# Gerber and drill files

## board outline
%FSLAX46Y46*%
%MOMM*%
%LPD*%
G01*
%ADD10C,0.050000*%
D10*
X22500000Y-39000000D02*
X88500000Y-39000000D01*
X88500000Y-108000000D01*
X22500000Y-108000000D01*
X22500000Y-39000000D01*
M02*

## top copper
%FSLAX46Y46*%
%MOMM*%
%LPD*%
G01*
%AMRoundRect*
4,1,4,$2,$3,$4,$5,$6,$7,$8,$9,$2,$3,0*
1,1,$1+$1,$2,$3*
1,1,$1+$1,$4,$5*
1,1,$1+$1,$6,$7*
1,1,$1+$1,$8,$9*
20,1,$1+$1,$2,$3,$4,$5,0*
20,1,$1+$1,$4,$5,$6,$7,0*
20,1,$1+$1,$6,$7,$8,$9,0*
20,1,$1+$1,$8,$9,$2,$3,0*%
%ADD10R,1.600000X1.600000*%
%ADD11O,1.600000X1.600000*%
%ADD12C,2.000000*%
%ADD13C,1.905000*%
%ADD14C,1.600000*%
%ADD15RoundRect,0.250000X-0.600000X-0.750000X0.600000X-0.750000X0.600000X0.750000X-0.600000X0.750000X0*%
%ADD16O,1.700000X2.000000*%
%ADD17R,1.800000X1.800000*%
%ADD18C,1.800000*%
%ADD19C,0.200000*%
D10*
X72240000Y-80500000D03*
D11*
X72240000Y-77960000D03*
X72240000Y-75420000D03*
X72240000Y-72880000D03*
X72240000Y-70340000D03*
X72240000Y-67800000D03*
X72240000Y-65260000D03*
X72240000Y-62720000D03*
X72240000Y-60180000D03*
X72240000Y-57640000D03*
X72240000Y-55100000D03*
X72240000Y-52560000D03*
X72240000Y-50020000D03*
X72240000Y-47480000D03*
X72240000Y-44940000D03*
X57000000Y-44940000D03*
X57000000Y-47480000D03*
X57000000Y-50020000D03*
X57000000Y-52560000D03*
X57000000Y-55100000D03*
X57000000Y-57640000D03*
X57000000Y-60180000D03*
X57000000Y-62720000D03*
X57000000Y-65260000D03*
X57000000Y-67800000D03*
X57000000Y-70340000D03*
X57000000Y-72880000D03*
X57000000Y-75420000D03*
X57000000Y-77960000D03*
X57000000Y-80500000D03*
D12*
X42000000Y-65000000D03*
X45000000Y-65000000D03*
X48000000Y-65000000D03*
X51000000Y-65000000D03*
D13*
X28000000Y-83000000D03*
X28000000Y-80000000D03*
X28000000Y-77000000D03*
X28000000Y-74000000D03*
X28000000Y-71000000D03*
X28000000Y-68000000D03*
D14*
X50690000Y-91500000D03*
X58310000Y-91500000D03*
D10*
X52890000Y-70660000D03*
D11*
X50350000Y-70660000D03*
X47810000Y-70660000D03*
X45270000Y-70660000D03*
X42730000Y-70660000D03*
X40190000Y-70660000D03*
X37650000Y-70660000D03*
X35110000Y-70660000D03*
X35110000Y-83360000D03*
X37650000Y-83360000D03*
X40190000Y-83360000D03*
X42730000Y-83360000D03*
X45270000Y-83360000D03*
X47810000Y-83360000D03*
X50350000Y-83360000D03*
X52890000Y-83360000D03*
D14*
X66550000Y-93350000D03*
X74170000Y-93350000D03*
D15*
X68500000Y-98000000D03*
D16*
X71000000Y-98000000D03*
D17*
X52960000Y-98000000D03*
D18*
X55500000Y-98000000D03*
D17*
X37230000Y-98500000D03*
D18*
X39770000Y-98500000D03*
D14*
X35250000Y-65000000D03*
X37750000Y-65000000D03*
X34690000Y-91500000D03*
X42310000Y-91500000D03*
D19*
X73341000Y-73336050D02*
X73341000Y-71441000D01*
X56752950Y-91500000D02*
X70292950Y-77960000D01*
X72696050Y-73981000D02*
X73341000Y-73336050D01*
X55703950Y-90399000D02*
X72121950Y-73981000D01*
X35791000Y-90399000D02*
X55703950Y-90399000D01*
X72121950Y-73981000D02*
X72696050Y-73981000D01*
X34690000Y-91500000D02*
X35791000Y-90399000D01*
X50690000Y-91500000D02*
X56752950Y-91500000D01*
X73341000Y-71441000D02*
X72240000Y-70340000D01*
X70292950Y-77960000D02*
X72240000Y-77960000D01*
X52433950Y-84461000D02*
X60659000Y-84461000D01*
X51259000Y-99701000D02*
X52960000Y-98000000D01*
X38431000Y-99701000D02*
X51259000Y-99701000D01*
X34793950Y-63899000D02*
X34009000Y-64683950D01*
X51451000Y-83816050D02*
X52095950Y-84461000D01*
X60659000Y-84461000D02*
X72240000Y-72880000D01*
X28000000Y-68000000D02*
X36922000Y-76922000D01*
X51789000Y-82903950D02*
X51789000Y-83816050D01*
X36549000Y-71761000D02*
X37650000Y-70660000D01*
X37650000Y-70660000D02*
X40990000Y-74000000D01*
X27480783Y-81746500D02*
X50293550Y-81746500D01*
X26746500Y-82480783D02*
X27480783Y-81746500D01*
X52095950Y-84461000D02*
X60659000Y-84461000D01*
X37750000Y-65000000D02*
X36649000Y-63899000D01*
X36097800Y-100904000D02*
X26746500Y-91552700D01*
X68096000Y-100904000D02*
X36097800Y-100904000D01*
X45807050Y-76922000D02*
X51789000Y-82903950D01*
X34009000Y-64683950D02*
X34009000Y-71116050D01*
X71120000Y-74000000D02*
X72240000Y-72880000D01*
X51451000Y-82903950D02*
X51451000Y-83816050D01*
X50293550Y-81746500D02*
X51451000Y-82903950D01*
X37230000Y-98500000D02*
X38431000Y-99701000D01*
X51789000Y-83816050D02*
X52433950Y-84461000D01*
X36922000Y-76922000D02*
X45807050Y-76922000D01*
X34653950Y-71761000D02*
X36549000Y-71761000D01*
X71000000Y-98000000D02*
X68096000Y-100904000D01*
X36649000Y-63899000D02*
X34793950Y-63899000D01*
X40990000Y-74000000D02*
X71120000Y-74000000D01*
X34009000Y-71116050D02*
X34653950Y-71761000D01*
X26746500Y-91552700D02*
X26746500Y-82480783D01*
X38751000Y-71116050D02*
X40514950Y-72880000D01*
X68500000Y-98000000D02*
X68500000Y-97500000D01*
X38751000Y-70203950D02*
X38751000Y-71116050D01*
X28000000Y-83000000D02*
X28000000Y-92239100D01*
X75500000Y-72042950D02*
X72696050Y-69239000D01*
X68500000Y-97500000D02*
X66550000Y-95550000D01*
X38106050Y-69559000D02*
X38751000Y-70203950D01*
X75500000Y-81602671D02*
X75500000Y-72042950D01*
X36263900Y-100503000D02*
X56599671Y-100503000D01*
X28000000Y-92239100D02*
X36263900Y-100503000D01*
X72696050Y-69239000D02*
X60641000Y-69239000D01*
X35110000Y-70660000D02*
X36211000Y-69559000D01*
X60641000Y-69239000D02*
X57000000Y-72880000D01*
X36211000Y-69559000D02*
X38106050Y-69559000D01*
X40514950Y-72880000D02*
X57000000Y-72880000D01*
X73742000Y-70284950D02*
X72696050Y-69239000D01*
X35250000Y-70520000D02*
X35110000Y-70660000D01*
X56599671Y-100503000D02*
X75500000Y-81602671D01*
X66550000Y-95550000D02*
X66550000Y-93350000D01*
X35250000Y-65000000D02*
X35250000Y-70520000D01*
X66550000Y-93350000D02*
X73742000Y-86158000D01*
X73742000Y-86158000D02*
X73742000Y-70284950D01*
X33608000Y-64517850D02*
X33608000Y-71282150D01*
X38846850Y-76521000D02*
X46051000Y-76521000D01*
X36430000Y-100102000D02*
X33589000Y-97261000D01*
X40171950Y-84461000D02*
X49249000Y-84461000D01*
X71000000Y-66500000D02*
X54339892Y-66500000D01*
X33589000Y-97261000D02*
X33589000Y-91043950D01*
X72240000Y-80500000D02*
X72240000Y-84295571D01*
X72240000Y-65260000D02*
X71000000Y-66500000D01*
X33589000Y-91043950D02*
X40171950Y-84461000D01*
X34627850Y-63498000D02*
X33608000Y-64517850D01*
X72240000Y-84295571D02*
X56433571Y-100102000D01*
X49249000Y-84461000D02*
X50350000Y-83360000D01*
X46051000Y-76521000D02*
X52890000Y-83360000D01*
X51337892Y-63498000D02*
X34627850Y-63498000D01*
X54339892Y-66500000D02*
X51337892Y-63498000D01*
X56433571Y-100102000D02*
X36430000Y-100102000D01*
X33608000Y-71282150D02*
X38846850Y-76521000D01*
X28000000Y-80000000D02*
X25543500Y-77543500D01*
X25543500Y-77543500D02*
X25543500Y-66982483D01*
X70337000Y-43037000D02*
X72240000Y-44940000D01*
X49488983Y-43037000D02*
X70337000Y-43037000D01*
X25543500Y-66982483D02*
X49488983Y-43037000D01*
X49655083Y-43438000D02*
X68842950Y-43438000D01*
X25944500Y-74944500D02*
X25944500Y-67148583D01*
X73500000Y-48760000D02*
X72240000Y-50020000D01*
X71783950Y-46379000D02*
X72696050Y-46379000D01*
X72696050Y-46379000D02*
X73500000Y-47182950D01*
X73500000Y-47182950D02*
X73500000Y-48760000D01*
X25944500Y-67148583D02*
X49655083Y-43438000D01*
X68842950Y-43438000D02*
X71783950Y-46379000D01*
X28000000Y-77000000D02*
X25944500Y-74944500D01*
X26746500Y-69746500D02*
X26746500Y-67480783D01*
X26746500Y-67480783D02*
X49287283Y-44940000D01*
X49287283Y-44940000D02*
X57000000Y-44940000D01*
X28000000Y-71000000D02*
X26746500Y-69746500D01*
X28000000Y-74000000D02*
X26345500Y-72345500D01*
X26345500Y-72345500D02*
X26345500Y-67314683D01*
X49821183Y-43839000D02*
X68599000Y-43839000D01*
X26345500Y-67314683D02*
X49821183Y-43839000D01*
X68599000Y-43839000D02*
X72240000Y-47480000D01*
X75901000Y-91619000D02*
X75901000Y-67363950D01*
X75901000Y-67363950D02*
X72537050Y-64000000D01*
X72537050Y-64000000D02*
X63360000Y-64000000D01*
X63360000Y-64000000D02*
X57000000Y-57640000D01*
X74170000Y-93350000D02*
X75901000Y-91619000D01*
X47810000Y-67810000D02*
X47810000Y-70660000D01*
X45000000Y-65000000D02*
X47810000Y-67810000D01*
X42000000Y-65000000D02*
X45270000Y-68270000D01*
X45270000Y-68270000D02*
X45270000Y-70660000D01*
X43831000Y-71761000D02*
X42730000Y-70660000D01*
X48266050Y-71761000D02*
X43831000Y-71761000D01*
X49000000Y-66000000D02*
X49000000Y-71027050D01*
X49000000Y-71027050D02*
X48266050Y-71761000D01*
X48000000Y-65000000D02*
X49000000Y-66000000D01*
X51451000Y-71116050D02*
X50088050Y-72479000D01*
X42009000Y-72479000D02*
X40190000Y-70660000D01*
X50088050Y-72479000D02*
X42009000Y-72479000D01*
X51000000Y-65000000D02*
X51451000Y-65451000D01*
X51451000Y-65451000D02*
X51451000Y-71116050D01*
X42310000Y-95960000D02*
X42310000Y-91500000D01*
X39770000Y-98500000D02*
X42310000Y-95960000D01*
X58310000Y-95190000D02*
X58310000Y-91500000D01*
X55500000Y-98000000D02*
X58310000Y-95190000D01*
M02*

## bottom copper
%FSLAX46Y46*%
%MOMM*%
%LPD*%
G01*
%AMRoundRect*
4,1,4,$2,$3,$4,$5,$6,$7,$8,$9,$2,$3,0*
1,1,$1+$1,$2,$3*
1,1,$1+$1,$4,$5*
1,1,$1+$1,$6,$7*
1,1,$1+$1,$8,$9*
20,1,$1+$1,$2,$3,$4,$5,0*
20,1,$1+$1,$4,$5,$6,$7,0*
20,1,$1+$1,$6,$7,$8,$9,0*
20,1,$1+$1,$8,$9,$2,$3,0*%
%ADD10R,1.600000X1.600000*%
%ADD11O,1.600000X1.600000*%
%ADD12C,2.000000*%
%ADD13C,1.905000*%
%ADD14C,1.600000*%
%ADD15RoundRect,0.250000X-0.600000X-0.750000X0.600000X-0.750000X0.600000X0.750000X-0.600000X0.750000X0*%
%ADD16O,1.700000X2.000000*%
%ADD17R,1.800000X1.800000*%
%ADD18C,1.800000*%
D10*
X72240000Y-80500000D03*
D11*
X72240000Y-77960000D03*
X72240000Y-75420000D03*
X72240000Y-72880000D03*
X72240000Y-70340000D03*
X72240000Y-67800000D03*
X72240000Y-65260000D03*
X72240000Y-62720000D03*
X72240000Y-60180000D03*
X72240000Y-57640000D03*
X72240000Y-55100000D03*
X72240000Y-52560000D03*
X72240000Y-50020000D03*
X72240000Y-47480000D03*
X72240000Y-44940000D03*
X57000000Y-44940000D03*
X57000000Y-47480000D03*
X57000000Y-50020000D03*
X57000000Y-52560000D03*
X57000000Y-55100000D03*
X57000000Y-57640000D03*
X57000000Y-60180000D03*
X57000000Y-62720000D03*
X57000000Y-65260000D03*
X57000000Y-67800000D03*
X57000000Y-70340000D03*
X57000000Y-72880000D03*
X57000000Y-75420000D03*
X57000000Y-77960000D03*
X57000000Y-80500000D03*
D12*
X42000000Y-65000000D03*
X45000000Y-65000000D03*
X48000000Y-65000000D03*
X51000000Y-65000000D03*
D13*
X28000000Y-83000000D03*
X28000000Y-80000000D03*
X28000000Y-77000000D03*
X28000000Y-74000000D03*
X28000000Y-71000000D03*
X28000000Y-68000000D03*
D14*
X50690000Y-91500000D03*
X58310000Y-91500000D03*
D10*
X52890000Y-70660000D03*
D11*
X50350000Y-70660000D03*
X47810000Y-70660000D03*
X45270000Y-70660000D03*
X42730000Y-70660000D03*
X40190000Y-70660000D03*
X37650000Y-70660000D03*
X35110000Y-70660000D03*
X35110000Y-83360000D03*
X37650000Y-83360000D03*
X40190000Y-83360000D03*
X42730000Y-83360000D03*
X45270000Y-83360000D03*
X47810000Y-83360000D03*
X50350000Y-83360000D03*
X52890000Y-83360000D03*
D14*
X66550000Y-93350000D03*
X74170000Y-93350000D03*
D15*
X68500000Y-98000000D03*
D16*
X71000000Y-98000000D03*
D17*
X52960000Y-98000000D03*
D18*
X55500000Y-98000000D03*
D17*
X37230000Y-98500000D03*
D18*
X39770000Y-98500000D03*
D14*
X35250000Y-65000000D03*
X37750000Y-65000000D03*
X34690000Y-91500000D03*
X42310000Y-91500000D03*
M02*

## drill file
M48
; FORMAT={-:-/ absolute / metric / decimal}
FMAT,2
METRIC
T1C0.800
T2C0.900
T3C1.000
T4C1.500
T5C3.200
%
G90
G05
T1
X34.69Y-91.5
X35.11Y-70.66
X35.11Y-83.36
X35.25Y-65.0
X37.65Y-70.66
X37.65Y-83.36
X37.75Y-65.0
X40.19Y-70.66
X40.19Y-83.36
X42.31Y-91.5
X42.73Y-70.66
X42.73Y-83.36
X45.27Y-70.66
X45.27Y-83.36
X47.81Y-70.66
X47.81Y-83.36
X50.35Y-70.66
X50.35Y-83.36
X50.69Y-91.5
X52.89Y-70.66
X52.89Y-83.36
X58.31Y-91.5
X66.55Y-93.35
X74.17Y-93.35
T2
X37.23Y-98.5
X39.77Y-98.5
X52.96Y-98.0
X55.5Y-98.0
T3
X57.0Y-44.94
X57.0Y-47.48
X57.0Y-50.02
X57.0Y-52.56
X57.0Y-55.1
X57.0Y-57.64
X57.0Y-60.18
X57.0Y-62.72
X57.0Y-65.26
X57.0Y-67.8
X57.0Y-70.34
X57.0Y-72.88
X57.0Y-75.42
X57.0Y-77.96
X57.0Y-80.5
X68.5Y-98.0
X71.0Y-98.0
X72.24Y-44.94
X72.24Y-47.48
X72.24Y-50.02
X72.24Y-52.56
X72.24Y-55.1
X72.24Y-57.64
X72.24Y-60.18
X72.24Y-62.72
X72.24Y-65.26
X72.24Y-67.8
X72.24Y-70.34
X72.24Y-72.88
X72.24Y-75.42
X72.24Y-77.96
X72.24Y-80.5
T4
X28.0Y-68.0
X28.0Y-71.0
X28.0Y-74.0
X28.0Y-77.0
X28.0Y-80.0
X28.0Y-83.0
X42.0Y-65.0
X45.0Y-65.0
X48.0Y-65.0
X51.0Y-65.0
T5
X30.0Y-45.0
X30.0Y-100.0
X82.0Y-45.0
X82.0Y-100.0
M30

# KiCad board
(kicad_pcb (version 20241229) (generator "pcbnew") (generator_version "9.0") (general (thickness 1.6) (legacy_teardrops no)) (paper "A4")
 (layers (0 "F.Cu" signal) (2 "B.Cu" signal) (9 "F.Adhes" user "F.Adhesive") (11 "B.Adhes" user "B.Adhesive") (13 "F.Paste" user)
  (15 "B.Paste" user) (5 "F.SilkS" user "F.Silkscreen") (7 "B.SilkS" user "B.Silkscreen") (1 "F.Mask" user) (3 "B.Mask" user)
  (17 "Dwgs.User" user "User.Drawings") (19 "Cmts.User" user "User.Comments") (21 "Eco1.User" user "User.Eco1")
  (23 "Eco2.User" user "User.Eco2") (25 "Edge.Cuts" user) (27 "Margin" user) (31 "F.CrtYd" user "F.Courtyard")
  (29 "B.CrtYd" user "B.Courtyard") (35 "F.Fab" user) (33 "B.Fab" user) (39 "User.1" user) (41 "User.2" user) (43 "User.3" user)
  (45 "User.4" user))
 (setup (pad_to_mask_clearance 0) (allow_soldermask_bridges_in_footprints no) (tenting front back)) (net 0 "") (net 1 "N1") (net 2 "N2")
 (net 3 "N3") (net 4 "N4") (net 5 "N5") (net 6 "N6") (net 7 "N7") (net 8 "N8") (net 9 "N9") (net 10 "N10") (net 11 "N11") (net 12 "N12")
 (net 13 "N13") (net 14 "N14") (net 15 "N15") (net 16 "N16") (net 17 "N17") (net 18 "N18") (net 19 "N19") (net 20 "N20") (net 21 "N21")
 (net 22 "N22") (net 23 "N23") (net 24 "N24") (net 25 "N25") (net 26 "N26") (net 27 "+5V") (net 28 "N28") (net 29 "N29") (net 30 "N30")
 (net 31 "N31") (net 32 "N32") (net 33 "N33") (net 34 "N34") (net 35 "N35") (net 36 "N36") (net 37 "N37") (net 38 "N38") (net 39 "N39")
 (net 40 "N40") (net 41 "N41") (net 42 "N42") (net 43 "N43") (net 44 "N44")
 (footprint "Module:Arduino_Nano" (layer "F.Cu") (at 72.24 80.5 180)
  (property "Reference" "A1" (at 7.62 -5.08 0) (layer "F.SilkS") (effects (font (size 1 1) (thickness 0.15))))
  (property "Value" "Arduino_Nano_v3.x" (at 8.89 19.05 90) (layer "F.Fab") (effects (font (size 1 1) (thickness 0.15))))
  (pad "1" thru_hole rect (at 0 0 180) (size 1.6 1.6) (drill 1) (layers "*.Cu" "*.Mask") (remove_unused_layers no) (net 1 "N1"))
  (pad "2" thru_hole oval (at 0 2.54 180) (size 1.6 1.6) (drill 1) (layers "*.Cu" "*.Mask") (remove_unused_layers no) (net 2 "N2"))
  (pad "3" thru_hole oval (at 0 5.08 180) (size 1.6 1.6) (drill 1) (layers "*.Cu" "*.Mask") (remove_unused_layers no) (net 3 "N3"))
  (pad "4" thru_hole oval (at 0 7.62 180) (size 1.6 1.6) (drill 1) (layers "*.Cu" "*.Mask") (remove_unused_layers no) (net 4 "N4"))
  (pad "5" thru_hole oval (at 0 10.16 180) (size 1.6 1.6) (drill 1) (layers "*.Cu" "*.Mask") (remove_unused_layers no) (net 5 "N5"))
  (pad "6" thru_hole oval (at 0 12.7 180) (size 1.6 1.6) (drill 1) (layers "*.Cu" "*.Mask") (remove_unused_layers no) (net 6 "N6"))
  (pad "7" thru_hole oval (at 0 15.24 180) (size 1.6 1.6) (drill 1) (layers "*.Cu" "*.Mask") (remove_unused_layers no) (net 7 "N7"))
  (pad "8" thru_hole oval (at 0 17.78 180) (size 1.6 1.6) (drill 1) (layers "*.Cu" "*.Mask") (remove_unused_layers no) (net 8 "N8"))
  (pad "9" thru_hole oval (at 0 20.32 180) (size 1.6 1.6) (drill 1) (layers "*.Cu" "*.Mask") (remove_unused_layers no) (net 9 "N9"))
  (pad "10" thru_hole oval (at 0 22.86 180) (size 1.6 1.6) (drill 1) (layers "*.Cu" "*.Mask") (remove_unused_layers no) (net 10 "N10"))
  (pad "11" thru_hole oval (at 0 25.4 180) (size 1.6 1.6) (drill 1) (layers "*.Cu" "*.Mask") (remove_unused_layers no) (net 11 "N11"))
  (pad "12" thru_hole oval (at 0 27.94 180) (size 1.6 1.6) (drill 1) (layers "*.Cu" "*.Mask") (remove_unused_layers no) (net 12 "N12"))
  (pad "13" thru_hole oval (at 0 30.48 180) (size 1.6 1.6) (drill 1) (layers "*.Cu" "*.Mask") (remove_unused_layers no) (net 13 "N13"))
  (pad "14" thru_hole oval (at 0 33.02 180) (size 1.6 1.6) (drill 1) (layers "*.Cu" "*.Mask") (remove_unused_layers no) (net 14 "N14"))
  (pad "15" thru_hole oval (at 0 35.56 180) (size 1.6 1.6) (drill 1) (layers "*.Cu" "*.Mask") (remove_unused_layers no) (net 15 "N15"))
  (pad "16" thru_hole oval (at 15.24 35.56 180) (size 1.6 1.6) (drill 1) (layers "*.Cu" "*.Mask") (remove_unused_layers no) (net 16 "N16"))
  (pad "17" thru_hole oval (at 15.24 33.02 180) (size 1.6 1.6) (drill 1) (layers "*.Cu" "*.Mask") (remove_unused_layers no) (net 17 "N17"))
  (pad "18" thru_hole oval (at 15.24 30.48 180) (size 1.6 1.6) (drill 1) (layers "*.Cu" "*.Mask") (remove_unused_layers no) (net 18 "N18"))
  (pad "19" thru_hole oval (at 15.24 27.94 180) (size 1.6 1.6) (drill 1) (layers "*.Cu" "*.Mask") (remove_unused_layers no) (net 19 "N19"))
  (pad "20" thru_hole oval (at 15.24 25.4 180) (size 1.6 1.6) (drill 1) (layers "*.Cu" "*.Mask") (remove_unused_layers no) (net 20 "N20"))
  (pad "21" thru_hole oval (at 15.24 22.86 180) (size 1.6 1.6) (drill 1) (layers "*.Cu" "*.Mask") (remove_unused_layers no) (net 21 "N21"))
  (pad "22" thru_hole oval (at 15.24 20.32 180) (size 1.6 1.6) (drill 1) (layers "*.Cu" "*.Mask") (remove_unused_layers no) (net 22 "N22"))
  (pad "23" thru_hole oval (at 15.24 17.78 180) (size 1.6 1.6) (drill 1) (layers "*.Cu" "*.Mask") (remove_unused_layers no) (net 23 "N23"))
  (pad "24" thru_hole oval (at 15.24 15.24 180) (size 1.6 1.6) (drill 1) (layers "*.Cu" "*.Mask") (remove_unused_layers no) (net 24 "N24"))
  (pad "25" thru_hole oval (at 15.24 12.7 180) (size 1.6 1.6) (drill 1) (layers "*.Cu" "*.Mask") (remove_unused_layers no) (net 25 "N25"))
  (pad "26" thru_hole oval (at 15.24 10.16 180) (size 1.6 1.6) (drill 1) (layers "*.Cu" "*.Mask") (remove_unused_layers no) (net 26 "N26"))
  (pad "27" thru_hole oval (at 15.24 7.62 180) (size 1.6 1.6) (drill 1) (layers "*.Cu" "*.Mask") (remove_unused_layers no) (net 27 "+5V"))
  (pad "28" thru_hole oval (at 15.24 5.08 180) (size 1.6 1.6) (drill 1) (layers "*.Cu" "*.Mask") (remove_unused_layers no) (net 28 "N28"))
  (pad "29" thru_hole oval (at 15.24 2.54 180) (size 1.6 1.6) (drill 1) (layers "*.Cu" "*.Mask") (remove_unused_layers no) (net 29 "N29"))
  (pad "30" thru_hole oval (at 15.24 0 180) (size 1.6 1.6) (drill 1) (layers "*.Cu" "*.Mask") (remove_unused_layers no) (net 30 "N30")))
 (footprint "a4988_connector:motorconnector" (layer "F.Cu") (at 52 70)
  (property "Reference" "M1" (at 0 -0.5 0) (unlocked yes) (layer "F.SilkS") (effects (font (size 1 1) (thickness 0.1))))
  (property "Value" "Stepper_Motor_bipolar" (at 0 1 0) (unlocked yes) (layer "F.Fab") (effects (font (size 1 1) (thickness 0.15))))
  (pad "1" thru_hole circle (at -10 -5) (size 2 2) (drill 1.5) (layers "*.Cu" "*.Mask") (remove_unused_layers no) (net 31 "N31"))
  (pad "2" thru_hole circle (at -7 -5) (size 2 2) (drill 1.5) (layers "*.Cu" "*.Mask") (remove_unused_layers no) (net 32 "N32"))
  (pad "3" thru_hole circle (at -4 -5) (size 2 2) (drill 1.5) (layers "*.Cu" "*.Mask") (remove_unused_layers no) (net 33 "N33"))
  (pad "4" thru_hole circle (at -1 -5) (size 2 2) (drill 1.5) (layers "*.Cu" "*.Mask" "F.Adhes") (remove_unused_layers no) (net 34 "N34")))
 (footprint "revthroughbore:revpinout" (layer "F.Cu") (at 30 76 90)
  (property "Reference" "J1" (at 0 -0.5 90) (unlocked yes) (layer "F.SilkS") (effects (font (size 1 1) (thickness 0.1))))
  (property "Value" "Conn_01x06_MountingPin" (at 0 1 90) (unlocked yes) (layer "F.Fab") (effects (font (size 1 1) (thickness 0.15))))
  (pad "1" thru_hole circle (at -7 -2 90) (size 1.905 1.905) (drill 1.5) (layers "*.Cu" "*.Mask") (remove_unused_layers no) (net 27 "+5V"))
  (pad "2" thru_hole circle (at -4 -2 90) (size 1.905 1.905) (drill 1.5) (layers "*.Cu" "*.Mask") (remove_unused_layers no) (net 15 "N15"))
  (pad "3" thru_hole circle (at -1 -2 90) (size 1.905 1.905) (drill 1.5) (layers "*.Cu" "*.Mask") (remove_unused_layers no) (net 13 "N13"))
  (pad "4" thru_hole circle (at 2 -2 90) (size 1.905 1.905) (drill 1.5) (layers "*.Cu" "*.Mask") (remove_unused_layers no) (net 14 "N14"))
  (pad "5" thru_hole circle (at 5 -2 90) (size 1.905 1.905) (drill 1.5) (layers "*.Cu" "*.Mask") (remove_unused_layers no) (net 16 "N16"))
  (pad "6" thru_hole circle (at 8 -2 90) (size 1.905 1.905) (drill 1.5) (layers "*.Cu" "*.Mask") (remove_unused_layers no) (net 4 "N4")))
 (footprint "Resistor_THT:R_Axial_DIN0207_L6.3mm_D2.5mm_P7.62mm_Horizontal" (layer "F.Cu") (at 50.69 91.5)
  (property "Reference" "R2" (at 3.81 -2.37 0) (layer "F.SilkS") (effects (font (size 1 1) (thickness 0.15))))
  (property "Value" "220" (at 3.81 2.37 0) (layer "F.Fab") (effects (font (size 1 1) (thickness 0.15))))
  (pad "1" thru_hole circle (at 0 0) (size 1.6 1.6) (drill 0.8) (layers "*.Cu" "*.Mask") (remove_unused_layers no) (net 19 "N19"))
  (pad "2" thru_hole circle (at 7.62 0) (size 1.6 1.6) (drill 0.8) (layers "*.Cu" "*.Mask") (remove_unused_layers no) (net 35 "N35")))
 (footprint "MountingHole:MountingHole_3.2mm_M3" (layer "F.Cu") (at 82 100)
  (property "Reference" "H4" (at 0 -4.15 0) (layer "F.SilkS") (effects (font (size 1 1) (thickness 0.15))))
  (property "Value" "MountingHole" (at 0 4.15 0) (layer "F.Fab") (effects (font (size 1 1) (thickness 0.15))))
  (pad "" np_thru_hole circle (at 0 0) (size 3.2 3.2) (drill 3.2) (layers "*.Cu" "*.Mask")))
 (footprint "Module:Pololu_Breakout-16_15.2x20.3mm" (layer "F.Cu") (at 52.89 70.66 -90)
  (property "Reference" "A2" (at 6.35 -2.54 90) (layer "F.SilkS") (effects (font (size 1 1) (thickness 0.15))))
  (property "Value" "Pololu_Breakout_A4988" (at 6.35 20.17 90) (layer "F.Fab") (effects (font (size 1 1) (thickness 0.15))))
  (pad "1" thru_hole rect (at 0 0 270) (size 1.6 1.6) (drill 0.8) (layers "*.Cu" "*.Mask") (remove_unused_layers no) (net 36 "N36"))
  (pad "2" thru_hole oval (at 0 2.54 270) (size 1.6 1.6) (drill 0.8) (layers "*.Cu" "*.Mask") (remove_unused_layers no) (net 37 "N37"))
  (pad "3" thru_hole oval (at 0 5.08 270) (size 1.6 1.6) (drill 0.8) (layers "*.Cu" "*.Mask") (remove_unused_layers no) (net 32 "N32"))
  (pad "4" thru_hole oval (at 0 7.62 270) (size 1.6 1.6) (drill 0.8) (layers "*.Cu" "*.Mask") (remove_unused_layers no) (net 31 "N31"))
  (pad "5" thru_hole oval (at 0 10.16 270) (size 1.6 1.6) (drill 0.8) (layers "*.Cu" "*.Mask") (remove_unused_layers no) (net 33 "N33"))
  (pad "6" thru_hole oval (at 0 12.7 270) (size 1.6 1.6) (drill 0.8) (layers "*.Cu" "*.Mask") (remove_unused_layers no) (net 34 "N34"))
  (pad "7" thru_hole oval (at 0 15.24 270) (size 1.6 1.6) (drill 0.8) (layers "*.Cu" "*.Mask") (remove_unused_layers no) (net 4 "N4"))
  (pad "8" thru_hole oval (at 0 17.78 270) (size 1.6 1.6) (drill 0.8) (layers "*.Cu" "*.Mask") (remove_unused_layers no) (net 27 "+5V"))
  (pad "9" thru_hole oval (at 12.7 17.78 270) (size 1.6 1.6) (drill 0.8) (layers "*.Cu" "*.Mask") (remove_unused_layers no) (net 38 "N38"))
  (pad "10" thru_hole oval (at 12.7 15.24 270) (size 1.6 1.6) (drill 0.8) (layers "*.Cu" "*.Mask") (remove_unused_layers no) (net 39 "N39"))
  (pad "11" thru_hole oval (at 12.7 12.7 270) (size 1.6 1.6) (drill 0.8) (layers "*.Cu" "*.Mask") (remove_unused_layers no) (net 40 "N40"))
  (pad "12" thru_hole oval (at 12.7 10.16 270) (size 1.6 1.6) (drill 0.8) (layers "*.Cu" "*.Mask") (remove_unused_layers no) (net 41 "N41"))
  (pad "13" thru_hole oval (at 12.7 7.62 270) (size 1.6 1.6) (drill 0.8) (layers "*.Cu" "*.Mask") (remove_unused_layers no) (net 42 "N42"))
  (pad "14" thru_hole oval (at 12.7 5.08 270) (size 1.6 1.6) (drill 0.8) (layers "*.Cu" "*.Mask") (remove_unused_layers no) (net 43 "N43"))
  (pad "15" thru_hole oval (at 12.7 2.54 270) (size 1.6 1.6) (drill 0.8) (layers "*.Cu" "*.Mask") (remove_unused_layers no) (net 7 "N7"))
  (pad "16" thru_hole oval (at 12.7 0 270) (size 1.6 1.6) (drill 0.8) (layers "*.Cu" "*.Mask") (remove_unused_layers no) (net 8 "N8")))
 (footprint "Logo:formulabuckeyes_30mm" (layer "F.Cu") (at 40 52.5)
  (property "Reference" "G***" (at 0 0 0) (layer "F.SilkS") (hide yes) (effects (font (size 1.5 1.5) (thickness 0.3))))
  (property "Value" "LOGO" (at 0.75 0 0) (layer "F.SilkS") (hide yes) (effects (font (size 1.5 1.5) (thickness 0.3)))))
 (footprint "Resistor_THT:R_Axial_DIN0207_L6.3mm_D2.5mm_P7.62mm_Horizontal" (layer "F.Cu") (at 66.55 93.35)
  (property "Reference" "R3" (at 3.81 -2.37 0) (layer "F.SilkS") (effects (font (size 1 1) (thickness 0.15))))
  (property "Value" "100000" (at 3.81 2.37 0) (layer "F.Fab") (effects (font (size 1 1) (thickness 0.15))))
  (pad "1" thru_hole circle (at 0 0) (size 1.6 1.6) (drill 0.8) (layers "*.Cu" "*.Mask") (remove_unused_layers no) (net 27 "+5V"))
  (pad "2" thru_hole circle (at 7.62 0) (size 1.6 1.6) (drill 0.8) (layers "*.Cu" "*.Mask") (remove_unused_layers no) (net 21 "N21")))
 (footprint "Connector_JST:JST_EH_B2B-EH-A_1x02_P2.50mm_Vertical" (layer "F.Cu") (at 68.5 98)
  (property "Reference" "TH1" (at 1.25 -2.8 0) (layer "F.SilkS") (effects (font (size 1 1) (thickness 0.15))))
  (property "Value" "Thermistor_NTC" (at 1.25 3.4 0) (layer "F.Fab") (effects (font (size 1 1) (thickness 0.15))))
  (pad "1" thru_hole roundrect (at 0 0) (size 1.7 2) (drill 1) (layers "*.Cu" "*.Mask") (remove_unused_layers no)
   (roundrect_rratio 0.147059) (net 27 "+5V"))
  (pad "2" thru_hole oval (at 2.5 0) (size 1.7 2) (drill 1) (layers "*.Cu" "*.Mask") (remove_unused_layers no) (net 4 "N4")))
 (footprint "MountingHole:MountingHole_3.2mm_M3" (layer "F.Cu") (at 82 45)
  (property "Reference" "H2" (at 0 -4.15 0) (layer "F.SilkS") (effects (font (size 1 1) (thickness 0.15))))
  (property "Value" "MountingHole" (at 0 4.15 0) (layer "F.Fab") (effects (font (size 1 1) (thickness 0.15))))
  (pad "" np_thru_hole circle (at 0 0) (size 3.2 3.2) (drill 3.2) (layers "*.Cu" "*.Mask")))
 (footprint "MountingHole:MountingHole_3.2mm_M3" (layer "F.Cu") (at 30 45)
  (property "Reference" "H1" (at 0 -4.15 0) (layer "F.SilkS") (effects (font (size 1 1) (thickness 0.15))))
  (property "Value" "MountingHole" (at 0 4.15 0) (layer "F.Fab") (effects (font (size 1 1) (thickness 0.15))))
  (pad "" np_thru_hole circle (at 0 0) (size 3.2 3.2) (drill 3.2) (layers "*.Cu" "*.Mask")))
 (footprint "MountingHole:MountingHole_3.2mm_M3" (layer "F.Cu") (at 30 100)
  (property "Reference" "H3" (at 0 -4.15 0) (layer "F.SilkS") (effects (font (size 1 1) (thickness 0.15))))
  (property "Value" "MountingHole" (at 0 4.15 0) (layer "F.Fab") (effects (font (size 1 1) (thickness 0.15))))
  (pad "" np_thru_hole circle (at 0 0) (size 3.2 3.2) (drill 3.2) (layers "*.Cu" "*.Mask")))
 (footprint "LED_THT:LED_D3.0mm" (layer "F.Cu") (at 52.96 98)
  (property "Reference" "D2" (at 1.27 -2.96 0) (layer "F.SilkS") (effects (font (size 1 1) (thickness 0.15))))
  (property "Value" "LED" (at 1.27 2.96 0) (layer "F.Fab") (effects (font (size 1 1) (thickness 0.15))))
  (pad "1" thru_hole rect (at 0 0) (size 1.8 1.8) (drill 0.9) (layers "*.Cu" "*.Mask") (remove_unused_layers no) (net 4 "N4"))
  (pad "2" thru_hole circle (at 2.54 0) (size 1.8 1.8) (drill 0.9) (layers "*.Cu" "*.Mask") (remove_unused_layers no) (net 35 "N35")))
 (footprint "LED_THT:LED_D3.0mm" (layer "F.Cu") (at 37.23 98.5)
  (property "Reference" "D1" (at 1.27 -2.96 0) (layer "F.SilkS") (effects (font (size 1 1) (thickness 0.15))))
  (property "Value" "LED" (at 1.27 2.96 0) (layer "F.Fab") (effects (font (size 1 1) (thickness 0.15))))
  (pad "1" thru_hole rect (at 0 0) (size 1.8 1.8) (drill 0.9) (layers "*.Cu" "*.Mask") (remove_unused_layers no) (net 4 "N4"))
  (pad "2" thru_hole circle (at 2.54 0) (size 1.8 1.8) (drill 0.9) (layers "*.Cu" "*.Mask") (remove_unused_layers no) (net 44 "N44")))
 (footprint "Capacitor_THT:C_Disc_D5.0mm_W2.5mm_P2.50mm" (layer "F.Cu") (at 35.25 65)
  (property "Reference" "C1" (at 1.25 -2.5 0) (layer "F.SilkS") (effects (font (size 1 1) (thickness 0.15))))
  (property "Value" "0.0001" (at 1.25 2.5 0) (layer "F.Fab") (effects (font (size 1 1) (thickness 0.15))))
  (pad "1" thru_hole circle (at 0 0) (size 1.6 1.6) (drill 0.8) (layers "*.Cu" "*.Mask") (remove_unused_layers no) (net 27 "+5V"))
  (pad "2" thru_hole circle (at 2.5 0) (size 1.6 1.6) (drill 0.8) (layers "*.Cu" "*.Mask") (remove_unused_layers no) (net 4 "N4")))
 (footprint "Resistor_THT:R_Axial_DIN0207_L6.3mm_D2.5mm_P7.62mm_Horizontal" (layer "F.Cu") (at 34.69 91.5)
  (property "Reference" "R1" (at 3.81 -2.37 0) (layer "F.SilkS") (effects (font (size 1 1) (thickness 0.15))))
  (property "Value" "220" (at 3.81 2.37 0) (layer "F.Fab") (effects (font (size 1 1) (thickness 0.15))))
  (pad "1" thru_hole circle (at 0 0) (size 1.6 1.6) (drill 0.8) (layers "*.Cu" "*.Mask") (remove_unused_layers no) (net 19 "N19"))
  (pad "2" thru_hole circle (at 7.62 0) (size 1.6 1.6) (drill 0.8) (layers "*.Cu" "*.Mask") (remove_unused_layers no) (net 44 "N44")))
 (gr_rect (start 22.5 39) (end 88.5 108) (stroke (width 0.05) (type default)) (fill no) (layer "Edge.Cuts"))
 (segment (start 73.341 73.33605) (end 73.341 71.441) (width 0.2) (layer "F.Cu") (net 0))
 (segment (start 56.75295 91.5) (end 70.29295 77.96) (width 0.2) (layer "F.Cu") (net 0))
 (segment (start 72.69605 73.981) (end 73.341 73.33605) (width 0.2) (layer "F.Cu") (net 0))
 (segment (start 55.70395 90.399) (end 72.12195 73.981) (width 0.2) (layer "F.Cu") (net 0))
 (segment (start 35.791 90.399) (end 55.70395 90.399) (width 0.2) (layer "F.Cu") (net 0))
 (segment (start 72.12195 73.981) (end 72.69605 73.981) (width 0.2) (layer "F.Cu") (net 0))
 (segment (start 34.69 91.5) (end 35.791 90.399) (width 0.2) (layer "F.Cu") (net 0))
 (segment (start 50.69 91.5) (end 56.75295 91.5) (width 0.2) (layer "F.Cu") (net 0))
 (segment (start 73.341 71.441) (end 72.24 70.34) (width 0.2) (layer "F.Cu") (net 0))
 (segment (start 70.29295 77.96) (end 72.24 77.96) (width 0.2) (layer "F.Cu") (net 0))
 (segment (start 52.43395 84.461) (end 60.659 84.461) (width 0.2) (layer "F.Cu") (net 4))
 (segment (start 51.259 99.701) (end 52.96 98) (width 0.2) (layer "F.Cu") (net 4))
 (segment (start 38.431 99.701) (end 51.259 99.701) (width 0.2) (layer "F.Cu") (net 4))
 (segment (start 34.79395 63.899) (end 34.009 64.68395) (width 0.2) (layer "F.Cu") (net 4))
 (segment (start 51.451 83.81605) (end 52.09595 84.461) (width 0.2) (layer "F.Cu") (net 4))
 (segment (start 60.659 84.461) (end 72.24 72.88) (width 0.2) (layer "F.Cu") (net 4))
 (segment (start 28 68) (end 36.922 76.922) (width 0.2) (layer "F.Cu") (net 4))
 (segment (start 51.789 82.90395) (end 51.789 83.81605) (width 0.2) (layer "F.Cu") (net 4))
 (segment (start 36.549 71.761) (end 37.65 70.66) (width 0.2) (layer "F.Cu") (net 4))
 (segment (start 37.65 70.66) (end 40.99 74) (width 0.2) (layer "F.Cu") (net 4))
 (segment (start 27.480783 81.7465) (end 50.29355 81.7465) (width 0.2) (layer "F.Cu") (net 4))
 (segment (start 26.7465 82.480783) (end 27.480783 81.7465) (width 0.2) (layer "F.Cu") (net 4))
 (segment (start 52.09595 84.461) (end 60.659 84.461) (width 0.2) (layer "F.Cu") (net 4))
 (segment (start 37.75 65) (end 36.649 63.899) (width 0.2) (layer "F.Cu") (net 4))
 (segment (start 36.0978 100.904) (end 26.7465 91.5527) (width 0.2) (layer "F.Cu") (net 4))
 (segment (start 68.096 100.904) (end 36.0978 100.904) (width 0.2) (layer "F.Cu") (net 4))
 (segment (start 45.80705 76.922) (end 51.789 82.90395) (width 0.2) (layer "F.Cu") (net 4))
 (segment (start 34.009 64.68395) (end 34.009 71.11605) (width 0.2) (layer "F.Cu") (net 4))
 (segment (start 71.12 74) (end 72.24 72.88) (width 0.2) (layer "F.Cu") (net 4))
 (segment (start 51.451 82.90395) (end 51.451 83.81605) (width 0.2) (layer "F.Cu") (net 4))
 (segment (start 50.29355 81.7465) (end 51.451 82.90395) (width 0.2) (layer "F.Cu") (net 4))
 (segment (start 37.23 98.5) (end 38.431 99.701) (width 0.2) (layer "F.Cu") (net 4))
 (segment (start 51.789 83.81605) (end 52.43395 84.461) (width 0.2) (layer "F.Cu") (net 4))
 (segment (start 36.922 76.922) (end 45.80705 76.922) (width 0.2) (layer "F.Cu") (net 4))
 (segment (start 34.65395 71.761) (end 36.549 71.761) (width 0.2) (layer "F.Cu") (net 4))
 (segment (start 71 98) (end 68.096 100.904) (width 0.2) (layer "F.Cu") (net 4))
 (segment (start 36.649 63.899) (end 34.79395 63.899) (width 0.2) (layer "F.Cu") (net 4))
 (segment (start 40.99 74) (end 71.12 74) (width 0.2) (layer "F.Cu") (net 4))
 (segment (start 34.009 71.11605) (end 34.65395 71.761) (width 0.2) (layer "F.Cu") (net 4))
 (segment (start 26.7465 91.5527) (end 26.7465 82.480783) (width 0.2) (layer "F.Cu") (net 4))
 (segment (start 38.751 71.11605) (end 40.51495 72.88) (width 0.2) (layer "F.Cu") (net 27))
 (segment (start 68.5 98) (end 68.5 97.5) (width 0.2) (layer "F.Cu") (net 27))
 (segment (start 38.751 70.20395) (end 38.751 71.11605) (width 0.2) (layer "F.Cu") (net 27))
 (segment (start 28 83) (end 28 92.2391) (width 0.2) (layer "F.Cu") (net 27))
 (segment (start 75.5 72.04295) (end 72.69605 69.239) (width 0.2) (layer "F.Cu") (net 27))
 (segment (start 68.5 97.5) (end 66.55 95.55) (width 0.2) (layer "F.Cu") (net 27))
 (segment (start 38.10605 69.559) (end 38.751 70.20395) (width 0.2) (layer "F.Cu") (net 27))
 (segment (start 75.5 81.602671) (end 75.5 72.04295) (width 0.2) (layer "F.Cu") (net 27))
 (segment (start 36.2639 100.503) (end 56.599671 100.503) (width 0.2) (layer "F.Cu") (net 27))
 (segment (start 28 92.2391) (end 36.2639 100.503) (width 0.2) (layer "F.Cu") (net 27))
 (segment (start 72.69605 69.239) (end 60.641 69.239) (width 0.2) (layer "F.Cu") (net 27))
 (segment (start 35.11 70.66) (end 36.211 69.559) (width 0.2) (layer "F.Cu") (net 27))
 (segment (start 60.641 69.239) (end 57 72.88) (width 0.2) (layer "F.Cu") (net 27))
 (segment (start 36.211 69.559) (end 38.10605 69.559) (width 0.2) (layer "F.Cu") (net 27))
 (segment (start 40.51495 72.88) (end 57 72.88) (width 0.2) (layer "F.Cu") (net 27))
 (segment (start 73.742 70.28495) (end 72.69605 69.239) (width 0.2) (layer "F.Cu") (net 27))
 (segment (start 35.25 70.52) (end 35.11 70.66) (width 0.2) (layer "F.Cu") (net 27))
 (segment (start 56.599671 100.503) (end 75.5 81.602671) (width 0.2) (layer "F.Cu") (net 27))
 (segment (start 66.55 95.55) (end 66.55 93.35) (width 0.2) (layer "F.Cu") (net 27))
 (segment (start 35.25 65) (end 35.25 70.52) (width 0.2) (layer "F.Cu") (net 27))
 (segment (start 66.55 93.35) (end 73.742 86.158) (width 0.2) (layer "F.Cu") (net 27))
 (segment (start 73.742 86.158) (end 73.742 70.28495) (width 0.2) (layer "F.Cu") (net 27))
 (segment (start 33.608 64.51785) (end 33.608 71.28215) (width 0.2) (layer "F.Cu") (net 7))
 (segment (start 38.84685 76.521) (end 46.051 76.521) (width 0.2) (layer "F.Cu") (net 7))
 (segment (start 36.43 100.102) (end 33.589 97.261) (width 0.2) (layer "F.Cu") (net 7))
 (segment (start 40.17195 84.461) (end 49.249 84.461) (width 0.2) (layer "F.Cu") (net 7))
 (segment (start 71 66.5) (end 54.339892 66.5) (width 0.2) (layer "F.Cu") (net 7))
 (segment (start 33.589 97.261) (end 33.589 91.04395) (width 0.2) (layer "F.Cu") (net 7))
 (segment (start 72.24 80.5) (end 72.24 84.295571) (width 0.2) (layer "F.Cu") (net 7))
 (segment (start 72.24 65.26) (end 71 66.5) (width 0.2) (layer "F.Cu") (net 7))
 (segment (start 33.589 91.04395) (end 40.17195 84.461) (width 0.2) (layer "F.Cu") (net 7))
 (segment (start 34.62785 63.498) (end 33.608 64.51785) (width 0.2) (layer "F.Cu") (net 7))
 (segment (start 72.24 84.295571) (end 56.433571 100.102) (width 0.2) (layer "F.Cu") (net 7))
 (segment (start 49.249 84.461) (end 50.35 83.36) (width 0.2) (layer "F.Cu") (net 7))
 (segment (start 46.051 76.521) (end 52.89 83.36) (width 0.2) (layer "F.Cu") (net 7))
 (segment (start 51.337892 63.498) (end 34.62785 63.498) (width 0.2) (layer "F.Cu") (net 7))
 (segment (start 54.339892 66.5) (end 51.337892 63.498) (width 0.2) (layer "F.Cu") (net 7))
 (segment (start 56.433571 100.102) (end 36.43 100.102) (width 0.2) (layer "F.Cu") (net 7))
 (segment (start 33.608 71.28215) (end 38.84685 76.521) (width 0.2) (layer "F.Cu") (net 7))
 (segment (start 28 80) (end 25.5435 77.5435) (width 0.2) (layer "F.Cu") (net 15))
 (segment (start 25.5435 77.5435) (end 25.5435 66.982483) (width 0.2) (layer "F.Cu") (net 15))
 (segment (start 70.337 43.037) (end 72.24 44.94) (width 0.2) (layer "F.Cu") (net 15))
 (segment (start 49.488983 43.037) (end 70.337 43.037) (width 0.2) (layer "F.Cu") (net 15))
 (segment (start 25.5435 66.982483) (end 49.488983 43.037) (width 0.2) (layer "F.Cu") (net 15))
 (segment (start 49.655083 43.438) (end 68.84295 43.438) (width 0.2) (layer "F.Cu") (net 13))
 (segment (start 25.9445 74.9445) (end 25.9445 67.148583) (width 0.2) (layer "F.Cu") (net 13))
 (segment (start 73.5 48.76) (end 72.24 50.02) (width 0.2) (layer "F.Cu") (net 13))
 (segment (start 71.78395 46.379) (end 72.69605 46.379) (width 0.2) (layer "F.Cu") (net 13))
 (segment (start 72.69605 46.379) (end 73.5 47.18295) (width 0.2) (layer "F.Cu") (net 13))
 (segment (start 73.5 47.18295) (end 73.5 48.76) (width 0.2) (layer "F.Cu") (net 13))
 (segment (start 25.9445 67.148583) (end 49.655083 43.438) (width 0.2) (layer "F.Cu") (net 13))
 (segment (start 68.84295 43.438) (end 71.78395 46.379) (width 0.2) (layer "F.Cu") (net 13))
 (segment (start 28 77) (end 25.9445 74.9445) (width 0.2) (layer "F.Cu") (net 13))
 (segment (start 26.7465 69.7465) (end 26.7465 67.480783) (width 0.2) (layer "F.Cu") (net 16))
 (segment (start 26.7465 67.480783) (end 49.287283 44.94) (width 0.2) (layer "F.Cu") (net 16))
 (segment (start 49.287283 44.94) (end 57 44.94) (width 0.2) (layer "F.Cu") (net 16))
 (segment (start 28 71) (end 26.7465 69.7465) (width 0.2) (layer "F.Cu") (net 16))
 (segment (start 28 74) (end 26.3455 72.3455) (width 0.2) (layer "F.Cu") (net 14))
 (segment (start 26.3455 72.3455) (end 26.3455 67.314683) (width 0.2) (layer "F.Cu") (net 14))
 (segment (start 49.821183 43.839) (end 68.599 43.839) (width 0.2) (layer "F.Cu") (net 14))
 (segment (start 26.3455 67.314683) (end 49.821183 43.839) (width 0.2) (layer "F.Cu") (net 14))
 (segment (start 68.599 43.839) (end 72.24 47.48) (width 0.2) (layer "F.Cu") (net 14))
 (segment (start 75.901 91.619) (end 75.901 67.36395) (width 0.2) (layer "F.Cu") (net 21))
 (segment (start 75.901 67.36395) (end 72.53705 64) (width 0.2) (layer "F.Cu") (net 21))
 (segment (start 72.53705 64) (end 63.36 64) (width 0.2) (layer "F.Cu") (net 21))
 (segment (start 63.36 64) (end 57 57.64) (width 0.2) (layer "F.Cu") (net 21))
 (segment (start 74.17 93.35) (end 75.901 91.619) (width 0.2) (layer "F.Cu") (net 21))
 (segment (start 47.81 67.81) (end 47.81 70.66) (width 0.2) (layer "F.Cu") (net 32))
 (segment (start 45 65) (end 47.81 67.81) (width 0.2) (layer "F.Cu") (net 32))
 (segment (start 42 65) (end 45.27 68.27) (width 0.2) (layer "F.Cu") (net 31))
 (segment (start 45.27 68.27) (end 45.27 70.66) (width 0.2) (layer "F.Cu") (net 31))
 (segment (start 43.831 71.761) (end 42.73 70.66) (width 0.2) (layer "F.Cu") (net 33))
 (segment (start 48.26605 71.761) (end 43.831 71.761) (width 0.2) (layer "F.Cu") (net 33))
 (segment (start 49 66) (end 49 71.02705) (width 0.2) (layer "F.Cu") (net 33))
 (segment (start 49 71.02705) (end 48.26605 71.761) (width 0.2) (layer "F.Cu") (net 33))
 (segment (start 48 65) (end 49 66) (width 0.2) (layer "F.Cu") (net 33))
 (segment (start 51.451 71.11605) (end 50.08805 72.479) (width 0.2) (layer "F.Cu") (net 34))
 (segment (start 42.009 72.479) (end 40.19 70.66) (width 0.2) (layer "F.Cu") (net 34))
 (segment (start 50.08805 72.479) (end 42.009 72.479) (width 0.2) (layer "F.Cu") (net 34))
 (segment (start 51 65) (end 51.451 65.451) (width 0.2) (layer "F.Cu") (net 34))
 (segment (start 51.451 65.451) (end 51.451 71.11605) (width 0.2) (layer "F.Cu") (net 34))
 (segment (start 42.31 95.96) (end 42.31 91.5) (width 0.2) (layer "F.Cu") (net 44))
 (segment (start 39.77 98.5) (end 42.31 95.96) (width 0.2) (layer "F.Cu") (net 44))
 (segment (start 58.31 95.19) (end 58.31 91.5) (width 0.2) (layer "F.Cu") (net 35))
 (segment (start 55.5 98) (end 58.31 95.19) (width 0.2) (layer "F.Cu") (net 35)))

